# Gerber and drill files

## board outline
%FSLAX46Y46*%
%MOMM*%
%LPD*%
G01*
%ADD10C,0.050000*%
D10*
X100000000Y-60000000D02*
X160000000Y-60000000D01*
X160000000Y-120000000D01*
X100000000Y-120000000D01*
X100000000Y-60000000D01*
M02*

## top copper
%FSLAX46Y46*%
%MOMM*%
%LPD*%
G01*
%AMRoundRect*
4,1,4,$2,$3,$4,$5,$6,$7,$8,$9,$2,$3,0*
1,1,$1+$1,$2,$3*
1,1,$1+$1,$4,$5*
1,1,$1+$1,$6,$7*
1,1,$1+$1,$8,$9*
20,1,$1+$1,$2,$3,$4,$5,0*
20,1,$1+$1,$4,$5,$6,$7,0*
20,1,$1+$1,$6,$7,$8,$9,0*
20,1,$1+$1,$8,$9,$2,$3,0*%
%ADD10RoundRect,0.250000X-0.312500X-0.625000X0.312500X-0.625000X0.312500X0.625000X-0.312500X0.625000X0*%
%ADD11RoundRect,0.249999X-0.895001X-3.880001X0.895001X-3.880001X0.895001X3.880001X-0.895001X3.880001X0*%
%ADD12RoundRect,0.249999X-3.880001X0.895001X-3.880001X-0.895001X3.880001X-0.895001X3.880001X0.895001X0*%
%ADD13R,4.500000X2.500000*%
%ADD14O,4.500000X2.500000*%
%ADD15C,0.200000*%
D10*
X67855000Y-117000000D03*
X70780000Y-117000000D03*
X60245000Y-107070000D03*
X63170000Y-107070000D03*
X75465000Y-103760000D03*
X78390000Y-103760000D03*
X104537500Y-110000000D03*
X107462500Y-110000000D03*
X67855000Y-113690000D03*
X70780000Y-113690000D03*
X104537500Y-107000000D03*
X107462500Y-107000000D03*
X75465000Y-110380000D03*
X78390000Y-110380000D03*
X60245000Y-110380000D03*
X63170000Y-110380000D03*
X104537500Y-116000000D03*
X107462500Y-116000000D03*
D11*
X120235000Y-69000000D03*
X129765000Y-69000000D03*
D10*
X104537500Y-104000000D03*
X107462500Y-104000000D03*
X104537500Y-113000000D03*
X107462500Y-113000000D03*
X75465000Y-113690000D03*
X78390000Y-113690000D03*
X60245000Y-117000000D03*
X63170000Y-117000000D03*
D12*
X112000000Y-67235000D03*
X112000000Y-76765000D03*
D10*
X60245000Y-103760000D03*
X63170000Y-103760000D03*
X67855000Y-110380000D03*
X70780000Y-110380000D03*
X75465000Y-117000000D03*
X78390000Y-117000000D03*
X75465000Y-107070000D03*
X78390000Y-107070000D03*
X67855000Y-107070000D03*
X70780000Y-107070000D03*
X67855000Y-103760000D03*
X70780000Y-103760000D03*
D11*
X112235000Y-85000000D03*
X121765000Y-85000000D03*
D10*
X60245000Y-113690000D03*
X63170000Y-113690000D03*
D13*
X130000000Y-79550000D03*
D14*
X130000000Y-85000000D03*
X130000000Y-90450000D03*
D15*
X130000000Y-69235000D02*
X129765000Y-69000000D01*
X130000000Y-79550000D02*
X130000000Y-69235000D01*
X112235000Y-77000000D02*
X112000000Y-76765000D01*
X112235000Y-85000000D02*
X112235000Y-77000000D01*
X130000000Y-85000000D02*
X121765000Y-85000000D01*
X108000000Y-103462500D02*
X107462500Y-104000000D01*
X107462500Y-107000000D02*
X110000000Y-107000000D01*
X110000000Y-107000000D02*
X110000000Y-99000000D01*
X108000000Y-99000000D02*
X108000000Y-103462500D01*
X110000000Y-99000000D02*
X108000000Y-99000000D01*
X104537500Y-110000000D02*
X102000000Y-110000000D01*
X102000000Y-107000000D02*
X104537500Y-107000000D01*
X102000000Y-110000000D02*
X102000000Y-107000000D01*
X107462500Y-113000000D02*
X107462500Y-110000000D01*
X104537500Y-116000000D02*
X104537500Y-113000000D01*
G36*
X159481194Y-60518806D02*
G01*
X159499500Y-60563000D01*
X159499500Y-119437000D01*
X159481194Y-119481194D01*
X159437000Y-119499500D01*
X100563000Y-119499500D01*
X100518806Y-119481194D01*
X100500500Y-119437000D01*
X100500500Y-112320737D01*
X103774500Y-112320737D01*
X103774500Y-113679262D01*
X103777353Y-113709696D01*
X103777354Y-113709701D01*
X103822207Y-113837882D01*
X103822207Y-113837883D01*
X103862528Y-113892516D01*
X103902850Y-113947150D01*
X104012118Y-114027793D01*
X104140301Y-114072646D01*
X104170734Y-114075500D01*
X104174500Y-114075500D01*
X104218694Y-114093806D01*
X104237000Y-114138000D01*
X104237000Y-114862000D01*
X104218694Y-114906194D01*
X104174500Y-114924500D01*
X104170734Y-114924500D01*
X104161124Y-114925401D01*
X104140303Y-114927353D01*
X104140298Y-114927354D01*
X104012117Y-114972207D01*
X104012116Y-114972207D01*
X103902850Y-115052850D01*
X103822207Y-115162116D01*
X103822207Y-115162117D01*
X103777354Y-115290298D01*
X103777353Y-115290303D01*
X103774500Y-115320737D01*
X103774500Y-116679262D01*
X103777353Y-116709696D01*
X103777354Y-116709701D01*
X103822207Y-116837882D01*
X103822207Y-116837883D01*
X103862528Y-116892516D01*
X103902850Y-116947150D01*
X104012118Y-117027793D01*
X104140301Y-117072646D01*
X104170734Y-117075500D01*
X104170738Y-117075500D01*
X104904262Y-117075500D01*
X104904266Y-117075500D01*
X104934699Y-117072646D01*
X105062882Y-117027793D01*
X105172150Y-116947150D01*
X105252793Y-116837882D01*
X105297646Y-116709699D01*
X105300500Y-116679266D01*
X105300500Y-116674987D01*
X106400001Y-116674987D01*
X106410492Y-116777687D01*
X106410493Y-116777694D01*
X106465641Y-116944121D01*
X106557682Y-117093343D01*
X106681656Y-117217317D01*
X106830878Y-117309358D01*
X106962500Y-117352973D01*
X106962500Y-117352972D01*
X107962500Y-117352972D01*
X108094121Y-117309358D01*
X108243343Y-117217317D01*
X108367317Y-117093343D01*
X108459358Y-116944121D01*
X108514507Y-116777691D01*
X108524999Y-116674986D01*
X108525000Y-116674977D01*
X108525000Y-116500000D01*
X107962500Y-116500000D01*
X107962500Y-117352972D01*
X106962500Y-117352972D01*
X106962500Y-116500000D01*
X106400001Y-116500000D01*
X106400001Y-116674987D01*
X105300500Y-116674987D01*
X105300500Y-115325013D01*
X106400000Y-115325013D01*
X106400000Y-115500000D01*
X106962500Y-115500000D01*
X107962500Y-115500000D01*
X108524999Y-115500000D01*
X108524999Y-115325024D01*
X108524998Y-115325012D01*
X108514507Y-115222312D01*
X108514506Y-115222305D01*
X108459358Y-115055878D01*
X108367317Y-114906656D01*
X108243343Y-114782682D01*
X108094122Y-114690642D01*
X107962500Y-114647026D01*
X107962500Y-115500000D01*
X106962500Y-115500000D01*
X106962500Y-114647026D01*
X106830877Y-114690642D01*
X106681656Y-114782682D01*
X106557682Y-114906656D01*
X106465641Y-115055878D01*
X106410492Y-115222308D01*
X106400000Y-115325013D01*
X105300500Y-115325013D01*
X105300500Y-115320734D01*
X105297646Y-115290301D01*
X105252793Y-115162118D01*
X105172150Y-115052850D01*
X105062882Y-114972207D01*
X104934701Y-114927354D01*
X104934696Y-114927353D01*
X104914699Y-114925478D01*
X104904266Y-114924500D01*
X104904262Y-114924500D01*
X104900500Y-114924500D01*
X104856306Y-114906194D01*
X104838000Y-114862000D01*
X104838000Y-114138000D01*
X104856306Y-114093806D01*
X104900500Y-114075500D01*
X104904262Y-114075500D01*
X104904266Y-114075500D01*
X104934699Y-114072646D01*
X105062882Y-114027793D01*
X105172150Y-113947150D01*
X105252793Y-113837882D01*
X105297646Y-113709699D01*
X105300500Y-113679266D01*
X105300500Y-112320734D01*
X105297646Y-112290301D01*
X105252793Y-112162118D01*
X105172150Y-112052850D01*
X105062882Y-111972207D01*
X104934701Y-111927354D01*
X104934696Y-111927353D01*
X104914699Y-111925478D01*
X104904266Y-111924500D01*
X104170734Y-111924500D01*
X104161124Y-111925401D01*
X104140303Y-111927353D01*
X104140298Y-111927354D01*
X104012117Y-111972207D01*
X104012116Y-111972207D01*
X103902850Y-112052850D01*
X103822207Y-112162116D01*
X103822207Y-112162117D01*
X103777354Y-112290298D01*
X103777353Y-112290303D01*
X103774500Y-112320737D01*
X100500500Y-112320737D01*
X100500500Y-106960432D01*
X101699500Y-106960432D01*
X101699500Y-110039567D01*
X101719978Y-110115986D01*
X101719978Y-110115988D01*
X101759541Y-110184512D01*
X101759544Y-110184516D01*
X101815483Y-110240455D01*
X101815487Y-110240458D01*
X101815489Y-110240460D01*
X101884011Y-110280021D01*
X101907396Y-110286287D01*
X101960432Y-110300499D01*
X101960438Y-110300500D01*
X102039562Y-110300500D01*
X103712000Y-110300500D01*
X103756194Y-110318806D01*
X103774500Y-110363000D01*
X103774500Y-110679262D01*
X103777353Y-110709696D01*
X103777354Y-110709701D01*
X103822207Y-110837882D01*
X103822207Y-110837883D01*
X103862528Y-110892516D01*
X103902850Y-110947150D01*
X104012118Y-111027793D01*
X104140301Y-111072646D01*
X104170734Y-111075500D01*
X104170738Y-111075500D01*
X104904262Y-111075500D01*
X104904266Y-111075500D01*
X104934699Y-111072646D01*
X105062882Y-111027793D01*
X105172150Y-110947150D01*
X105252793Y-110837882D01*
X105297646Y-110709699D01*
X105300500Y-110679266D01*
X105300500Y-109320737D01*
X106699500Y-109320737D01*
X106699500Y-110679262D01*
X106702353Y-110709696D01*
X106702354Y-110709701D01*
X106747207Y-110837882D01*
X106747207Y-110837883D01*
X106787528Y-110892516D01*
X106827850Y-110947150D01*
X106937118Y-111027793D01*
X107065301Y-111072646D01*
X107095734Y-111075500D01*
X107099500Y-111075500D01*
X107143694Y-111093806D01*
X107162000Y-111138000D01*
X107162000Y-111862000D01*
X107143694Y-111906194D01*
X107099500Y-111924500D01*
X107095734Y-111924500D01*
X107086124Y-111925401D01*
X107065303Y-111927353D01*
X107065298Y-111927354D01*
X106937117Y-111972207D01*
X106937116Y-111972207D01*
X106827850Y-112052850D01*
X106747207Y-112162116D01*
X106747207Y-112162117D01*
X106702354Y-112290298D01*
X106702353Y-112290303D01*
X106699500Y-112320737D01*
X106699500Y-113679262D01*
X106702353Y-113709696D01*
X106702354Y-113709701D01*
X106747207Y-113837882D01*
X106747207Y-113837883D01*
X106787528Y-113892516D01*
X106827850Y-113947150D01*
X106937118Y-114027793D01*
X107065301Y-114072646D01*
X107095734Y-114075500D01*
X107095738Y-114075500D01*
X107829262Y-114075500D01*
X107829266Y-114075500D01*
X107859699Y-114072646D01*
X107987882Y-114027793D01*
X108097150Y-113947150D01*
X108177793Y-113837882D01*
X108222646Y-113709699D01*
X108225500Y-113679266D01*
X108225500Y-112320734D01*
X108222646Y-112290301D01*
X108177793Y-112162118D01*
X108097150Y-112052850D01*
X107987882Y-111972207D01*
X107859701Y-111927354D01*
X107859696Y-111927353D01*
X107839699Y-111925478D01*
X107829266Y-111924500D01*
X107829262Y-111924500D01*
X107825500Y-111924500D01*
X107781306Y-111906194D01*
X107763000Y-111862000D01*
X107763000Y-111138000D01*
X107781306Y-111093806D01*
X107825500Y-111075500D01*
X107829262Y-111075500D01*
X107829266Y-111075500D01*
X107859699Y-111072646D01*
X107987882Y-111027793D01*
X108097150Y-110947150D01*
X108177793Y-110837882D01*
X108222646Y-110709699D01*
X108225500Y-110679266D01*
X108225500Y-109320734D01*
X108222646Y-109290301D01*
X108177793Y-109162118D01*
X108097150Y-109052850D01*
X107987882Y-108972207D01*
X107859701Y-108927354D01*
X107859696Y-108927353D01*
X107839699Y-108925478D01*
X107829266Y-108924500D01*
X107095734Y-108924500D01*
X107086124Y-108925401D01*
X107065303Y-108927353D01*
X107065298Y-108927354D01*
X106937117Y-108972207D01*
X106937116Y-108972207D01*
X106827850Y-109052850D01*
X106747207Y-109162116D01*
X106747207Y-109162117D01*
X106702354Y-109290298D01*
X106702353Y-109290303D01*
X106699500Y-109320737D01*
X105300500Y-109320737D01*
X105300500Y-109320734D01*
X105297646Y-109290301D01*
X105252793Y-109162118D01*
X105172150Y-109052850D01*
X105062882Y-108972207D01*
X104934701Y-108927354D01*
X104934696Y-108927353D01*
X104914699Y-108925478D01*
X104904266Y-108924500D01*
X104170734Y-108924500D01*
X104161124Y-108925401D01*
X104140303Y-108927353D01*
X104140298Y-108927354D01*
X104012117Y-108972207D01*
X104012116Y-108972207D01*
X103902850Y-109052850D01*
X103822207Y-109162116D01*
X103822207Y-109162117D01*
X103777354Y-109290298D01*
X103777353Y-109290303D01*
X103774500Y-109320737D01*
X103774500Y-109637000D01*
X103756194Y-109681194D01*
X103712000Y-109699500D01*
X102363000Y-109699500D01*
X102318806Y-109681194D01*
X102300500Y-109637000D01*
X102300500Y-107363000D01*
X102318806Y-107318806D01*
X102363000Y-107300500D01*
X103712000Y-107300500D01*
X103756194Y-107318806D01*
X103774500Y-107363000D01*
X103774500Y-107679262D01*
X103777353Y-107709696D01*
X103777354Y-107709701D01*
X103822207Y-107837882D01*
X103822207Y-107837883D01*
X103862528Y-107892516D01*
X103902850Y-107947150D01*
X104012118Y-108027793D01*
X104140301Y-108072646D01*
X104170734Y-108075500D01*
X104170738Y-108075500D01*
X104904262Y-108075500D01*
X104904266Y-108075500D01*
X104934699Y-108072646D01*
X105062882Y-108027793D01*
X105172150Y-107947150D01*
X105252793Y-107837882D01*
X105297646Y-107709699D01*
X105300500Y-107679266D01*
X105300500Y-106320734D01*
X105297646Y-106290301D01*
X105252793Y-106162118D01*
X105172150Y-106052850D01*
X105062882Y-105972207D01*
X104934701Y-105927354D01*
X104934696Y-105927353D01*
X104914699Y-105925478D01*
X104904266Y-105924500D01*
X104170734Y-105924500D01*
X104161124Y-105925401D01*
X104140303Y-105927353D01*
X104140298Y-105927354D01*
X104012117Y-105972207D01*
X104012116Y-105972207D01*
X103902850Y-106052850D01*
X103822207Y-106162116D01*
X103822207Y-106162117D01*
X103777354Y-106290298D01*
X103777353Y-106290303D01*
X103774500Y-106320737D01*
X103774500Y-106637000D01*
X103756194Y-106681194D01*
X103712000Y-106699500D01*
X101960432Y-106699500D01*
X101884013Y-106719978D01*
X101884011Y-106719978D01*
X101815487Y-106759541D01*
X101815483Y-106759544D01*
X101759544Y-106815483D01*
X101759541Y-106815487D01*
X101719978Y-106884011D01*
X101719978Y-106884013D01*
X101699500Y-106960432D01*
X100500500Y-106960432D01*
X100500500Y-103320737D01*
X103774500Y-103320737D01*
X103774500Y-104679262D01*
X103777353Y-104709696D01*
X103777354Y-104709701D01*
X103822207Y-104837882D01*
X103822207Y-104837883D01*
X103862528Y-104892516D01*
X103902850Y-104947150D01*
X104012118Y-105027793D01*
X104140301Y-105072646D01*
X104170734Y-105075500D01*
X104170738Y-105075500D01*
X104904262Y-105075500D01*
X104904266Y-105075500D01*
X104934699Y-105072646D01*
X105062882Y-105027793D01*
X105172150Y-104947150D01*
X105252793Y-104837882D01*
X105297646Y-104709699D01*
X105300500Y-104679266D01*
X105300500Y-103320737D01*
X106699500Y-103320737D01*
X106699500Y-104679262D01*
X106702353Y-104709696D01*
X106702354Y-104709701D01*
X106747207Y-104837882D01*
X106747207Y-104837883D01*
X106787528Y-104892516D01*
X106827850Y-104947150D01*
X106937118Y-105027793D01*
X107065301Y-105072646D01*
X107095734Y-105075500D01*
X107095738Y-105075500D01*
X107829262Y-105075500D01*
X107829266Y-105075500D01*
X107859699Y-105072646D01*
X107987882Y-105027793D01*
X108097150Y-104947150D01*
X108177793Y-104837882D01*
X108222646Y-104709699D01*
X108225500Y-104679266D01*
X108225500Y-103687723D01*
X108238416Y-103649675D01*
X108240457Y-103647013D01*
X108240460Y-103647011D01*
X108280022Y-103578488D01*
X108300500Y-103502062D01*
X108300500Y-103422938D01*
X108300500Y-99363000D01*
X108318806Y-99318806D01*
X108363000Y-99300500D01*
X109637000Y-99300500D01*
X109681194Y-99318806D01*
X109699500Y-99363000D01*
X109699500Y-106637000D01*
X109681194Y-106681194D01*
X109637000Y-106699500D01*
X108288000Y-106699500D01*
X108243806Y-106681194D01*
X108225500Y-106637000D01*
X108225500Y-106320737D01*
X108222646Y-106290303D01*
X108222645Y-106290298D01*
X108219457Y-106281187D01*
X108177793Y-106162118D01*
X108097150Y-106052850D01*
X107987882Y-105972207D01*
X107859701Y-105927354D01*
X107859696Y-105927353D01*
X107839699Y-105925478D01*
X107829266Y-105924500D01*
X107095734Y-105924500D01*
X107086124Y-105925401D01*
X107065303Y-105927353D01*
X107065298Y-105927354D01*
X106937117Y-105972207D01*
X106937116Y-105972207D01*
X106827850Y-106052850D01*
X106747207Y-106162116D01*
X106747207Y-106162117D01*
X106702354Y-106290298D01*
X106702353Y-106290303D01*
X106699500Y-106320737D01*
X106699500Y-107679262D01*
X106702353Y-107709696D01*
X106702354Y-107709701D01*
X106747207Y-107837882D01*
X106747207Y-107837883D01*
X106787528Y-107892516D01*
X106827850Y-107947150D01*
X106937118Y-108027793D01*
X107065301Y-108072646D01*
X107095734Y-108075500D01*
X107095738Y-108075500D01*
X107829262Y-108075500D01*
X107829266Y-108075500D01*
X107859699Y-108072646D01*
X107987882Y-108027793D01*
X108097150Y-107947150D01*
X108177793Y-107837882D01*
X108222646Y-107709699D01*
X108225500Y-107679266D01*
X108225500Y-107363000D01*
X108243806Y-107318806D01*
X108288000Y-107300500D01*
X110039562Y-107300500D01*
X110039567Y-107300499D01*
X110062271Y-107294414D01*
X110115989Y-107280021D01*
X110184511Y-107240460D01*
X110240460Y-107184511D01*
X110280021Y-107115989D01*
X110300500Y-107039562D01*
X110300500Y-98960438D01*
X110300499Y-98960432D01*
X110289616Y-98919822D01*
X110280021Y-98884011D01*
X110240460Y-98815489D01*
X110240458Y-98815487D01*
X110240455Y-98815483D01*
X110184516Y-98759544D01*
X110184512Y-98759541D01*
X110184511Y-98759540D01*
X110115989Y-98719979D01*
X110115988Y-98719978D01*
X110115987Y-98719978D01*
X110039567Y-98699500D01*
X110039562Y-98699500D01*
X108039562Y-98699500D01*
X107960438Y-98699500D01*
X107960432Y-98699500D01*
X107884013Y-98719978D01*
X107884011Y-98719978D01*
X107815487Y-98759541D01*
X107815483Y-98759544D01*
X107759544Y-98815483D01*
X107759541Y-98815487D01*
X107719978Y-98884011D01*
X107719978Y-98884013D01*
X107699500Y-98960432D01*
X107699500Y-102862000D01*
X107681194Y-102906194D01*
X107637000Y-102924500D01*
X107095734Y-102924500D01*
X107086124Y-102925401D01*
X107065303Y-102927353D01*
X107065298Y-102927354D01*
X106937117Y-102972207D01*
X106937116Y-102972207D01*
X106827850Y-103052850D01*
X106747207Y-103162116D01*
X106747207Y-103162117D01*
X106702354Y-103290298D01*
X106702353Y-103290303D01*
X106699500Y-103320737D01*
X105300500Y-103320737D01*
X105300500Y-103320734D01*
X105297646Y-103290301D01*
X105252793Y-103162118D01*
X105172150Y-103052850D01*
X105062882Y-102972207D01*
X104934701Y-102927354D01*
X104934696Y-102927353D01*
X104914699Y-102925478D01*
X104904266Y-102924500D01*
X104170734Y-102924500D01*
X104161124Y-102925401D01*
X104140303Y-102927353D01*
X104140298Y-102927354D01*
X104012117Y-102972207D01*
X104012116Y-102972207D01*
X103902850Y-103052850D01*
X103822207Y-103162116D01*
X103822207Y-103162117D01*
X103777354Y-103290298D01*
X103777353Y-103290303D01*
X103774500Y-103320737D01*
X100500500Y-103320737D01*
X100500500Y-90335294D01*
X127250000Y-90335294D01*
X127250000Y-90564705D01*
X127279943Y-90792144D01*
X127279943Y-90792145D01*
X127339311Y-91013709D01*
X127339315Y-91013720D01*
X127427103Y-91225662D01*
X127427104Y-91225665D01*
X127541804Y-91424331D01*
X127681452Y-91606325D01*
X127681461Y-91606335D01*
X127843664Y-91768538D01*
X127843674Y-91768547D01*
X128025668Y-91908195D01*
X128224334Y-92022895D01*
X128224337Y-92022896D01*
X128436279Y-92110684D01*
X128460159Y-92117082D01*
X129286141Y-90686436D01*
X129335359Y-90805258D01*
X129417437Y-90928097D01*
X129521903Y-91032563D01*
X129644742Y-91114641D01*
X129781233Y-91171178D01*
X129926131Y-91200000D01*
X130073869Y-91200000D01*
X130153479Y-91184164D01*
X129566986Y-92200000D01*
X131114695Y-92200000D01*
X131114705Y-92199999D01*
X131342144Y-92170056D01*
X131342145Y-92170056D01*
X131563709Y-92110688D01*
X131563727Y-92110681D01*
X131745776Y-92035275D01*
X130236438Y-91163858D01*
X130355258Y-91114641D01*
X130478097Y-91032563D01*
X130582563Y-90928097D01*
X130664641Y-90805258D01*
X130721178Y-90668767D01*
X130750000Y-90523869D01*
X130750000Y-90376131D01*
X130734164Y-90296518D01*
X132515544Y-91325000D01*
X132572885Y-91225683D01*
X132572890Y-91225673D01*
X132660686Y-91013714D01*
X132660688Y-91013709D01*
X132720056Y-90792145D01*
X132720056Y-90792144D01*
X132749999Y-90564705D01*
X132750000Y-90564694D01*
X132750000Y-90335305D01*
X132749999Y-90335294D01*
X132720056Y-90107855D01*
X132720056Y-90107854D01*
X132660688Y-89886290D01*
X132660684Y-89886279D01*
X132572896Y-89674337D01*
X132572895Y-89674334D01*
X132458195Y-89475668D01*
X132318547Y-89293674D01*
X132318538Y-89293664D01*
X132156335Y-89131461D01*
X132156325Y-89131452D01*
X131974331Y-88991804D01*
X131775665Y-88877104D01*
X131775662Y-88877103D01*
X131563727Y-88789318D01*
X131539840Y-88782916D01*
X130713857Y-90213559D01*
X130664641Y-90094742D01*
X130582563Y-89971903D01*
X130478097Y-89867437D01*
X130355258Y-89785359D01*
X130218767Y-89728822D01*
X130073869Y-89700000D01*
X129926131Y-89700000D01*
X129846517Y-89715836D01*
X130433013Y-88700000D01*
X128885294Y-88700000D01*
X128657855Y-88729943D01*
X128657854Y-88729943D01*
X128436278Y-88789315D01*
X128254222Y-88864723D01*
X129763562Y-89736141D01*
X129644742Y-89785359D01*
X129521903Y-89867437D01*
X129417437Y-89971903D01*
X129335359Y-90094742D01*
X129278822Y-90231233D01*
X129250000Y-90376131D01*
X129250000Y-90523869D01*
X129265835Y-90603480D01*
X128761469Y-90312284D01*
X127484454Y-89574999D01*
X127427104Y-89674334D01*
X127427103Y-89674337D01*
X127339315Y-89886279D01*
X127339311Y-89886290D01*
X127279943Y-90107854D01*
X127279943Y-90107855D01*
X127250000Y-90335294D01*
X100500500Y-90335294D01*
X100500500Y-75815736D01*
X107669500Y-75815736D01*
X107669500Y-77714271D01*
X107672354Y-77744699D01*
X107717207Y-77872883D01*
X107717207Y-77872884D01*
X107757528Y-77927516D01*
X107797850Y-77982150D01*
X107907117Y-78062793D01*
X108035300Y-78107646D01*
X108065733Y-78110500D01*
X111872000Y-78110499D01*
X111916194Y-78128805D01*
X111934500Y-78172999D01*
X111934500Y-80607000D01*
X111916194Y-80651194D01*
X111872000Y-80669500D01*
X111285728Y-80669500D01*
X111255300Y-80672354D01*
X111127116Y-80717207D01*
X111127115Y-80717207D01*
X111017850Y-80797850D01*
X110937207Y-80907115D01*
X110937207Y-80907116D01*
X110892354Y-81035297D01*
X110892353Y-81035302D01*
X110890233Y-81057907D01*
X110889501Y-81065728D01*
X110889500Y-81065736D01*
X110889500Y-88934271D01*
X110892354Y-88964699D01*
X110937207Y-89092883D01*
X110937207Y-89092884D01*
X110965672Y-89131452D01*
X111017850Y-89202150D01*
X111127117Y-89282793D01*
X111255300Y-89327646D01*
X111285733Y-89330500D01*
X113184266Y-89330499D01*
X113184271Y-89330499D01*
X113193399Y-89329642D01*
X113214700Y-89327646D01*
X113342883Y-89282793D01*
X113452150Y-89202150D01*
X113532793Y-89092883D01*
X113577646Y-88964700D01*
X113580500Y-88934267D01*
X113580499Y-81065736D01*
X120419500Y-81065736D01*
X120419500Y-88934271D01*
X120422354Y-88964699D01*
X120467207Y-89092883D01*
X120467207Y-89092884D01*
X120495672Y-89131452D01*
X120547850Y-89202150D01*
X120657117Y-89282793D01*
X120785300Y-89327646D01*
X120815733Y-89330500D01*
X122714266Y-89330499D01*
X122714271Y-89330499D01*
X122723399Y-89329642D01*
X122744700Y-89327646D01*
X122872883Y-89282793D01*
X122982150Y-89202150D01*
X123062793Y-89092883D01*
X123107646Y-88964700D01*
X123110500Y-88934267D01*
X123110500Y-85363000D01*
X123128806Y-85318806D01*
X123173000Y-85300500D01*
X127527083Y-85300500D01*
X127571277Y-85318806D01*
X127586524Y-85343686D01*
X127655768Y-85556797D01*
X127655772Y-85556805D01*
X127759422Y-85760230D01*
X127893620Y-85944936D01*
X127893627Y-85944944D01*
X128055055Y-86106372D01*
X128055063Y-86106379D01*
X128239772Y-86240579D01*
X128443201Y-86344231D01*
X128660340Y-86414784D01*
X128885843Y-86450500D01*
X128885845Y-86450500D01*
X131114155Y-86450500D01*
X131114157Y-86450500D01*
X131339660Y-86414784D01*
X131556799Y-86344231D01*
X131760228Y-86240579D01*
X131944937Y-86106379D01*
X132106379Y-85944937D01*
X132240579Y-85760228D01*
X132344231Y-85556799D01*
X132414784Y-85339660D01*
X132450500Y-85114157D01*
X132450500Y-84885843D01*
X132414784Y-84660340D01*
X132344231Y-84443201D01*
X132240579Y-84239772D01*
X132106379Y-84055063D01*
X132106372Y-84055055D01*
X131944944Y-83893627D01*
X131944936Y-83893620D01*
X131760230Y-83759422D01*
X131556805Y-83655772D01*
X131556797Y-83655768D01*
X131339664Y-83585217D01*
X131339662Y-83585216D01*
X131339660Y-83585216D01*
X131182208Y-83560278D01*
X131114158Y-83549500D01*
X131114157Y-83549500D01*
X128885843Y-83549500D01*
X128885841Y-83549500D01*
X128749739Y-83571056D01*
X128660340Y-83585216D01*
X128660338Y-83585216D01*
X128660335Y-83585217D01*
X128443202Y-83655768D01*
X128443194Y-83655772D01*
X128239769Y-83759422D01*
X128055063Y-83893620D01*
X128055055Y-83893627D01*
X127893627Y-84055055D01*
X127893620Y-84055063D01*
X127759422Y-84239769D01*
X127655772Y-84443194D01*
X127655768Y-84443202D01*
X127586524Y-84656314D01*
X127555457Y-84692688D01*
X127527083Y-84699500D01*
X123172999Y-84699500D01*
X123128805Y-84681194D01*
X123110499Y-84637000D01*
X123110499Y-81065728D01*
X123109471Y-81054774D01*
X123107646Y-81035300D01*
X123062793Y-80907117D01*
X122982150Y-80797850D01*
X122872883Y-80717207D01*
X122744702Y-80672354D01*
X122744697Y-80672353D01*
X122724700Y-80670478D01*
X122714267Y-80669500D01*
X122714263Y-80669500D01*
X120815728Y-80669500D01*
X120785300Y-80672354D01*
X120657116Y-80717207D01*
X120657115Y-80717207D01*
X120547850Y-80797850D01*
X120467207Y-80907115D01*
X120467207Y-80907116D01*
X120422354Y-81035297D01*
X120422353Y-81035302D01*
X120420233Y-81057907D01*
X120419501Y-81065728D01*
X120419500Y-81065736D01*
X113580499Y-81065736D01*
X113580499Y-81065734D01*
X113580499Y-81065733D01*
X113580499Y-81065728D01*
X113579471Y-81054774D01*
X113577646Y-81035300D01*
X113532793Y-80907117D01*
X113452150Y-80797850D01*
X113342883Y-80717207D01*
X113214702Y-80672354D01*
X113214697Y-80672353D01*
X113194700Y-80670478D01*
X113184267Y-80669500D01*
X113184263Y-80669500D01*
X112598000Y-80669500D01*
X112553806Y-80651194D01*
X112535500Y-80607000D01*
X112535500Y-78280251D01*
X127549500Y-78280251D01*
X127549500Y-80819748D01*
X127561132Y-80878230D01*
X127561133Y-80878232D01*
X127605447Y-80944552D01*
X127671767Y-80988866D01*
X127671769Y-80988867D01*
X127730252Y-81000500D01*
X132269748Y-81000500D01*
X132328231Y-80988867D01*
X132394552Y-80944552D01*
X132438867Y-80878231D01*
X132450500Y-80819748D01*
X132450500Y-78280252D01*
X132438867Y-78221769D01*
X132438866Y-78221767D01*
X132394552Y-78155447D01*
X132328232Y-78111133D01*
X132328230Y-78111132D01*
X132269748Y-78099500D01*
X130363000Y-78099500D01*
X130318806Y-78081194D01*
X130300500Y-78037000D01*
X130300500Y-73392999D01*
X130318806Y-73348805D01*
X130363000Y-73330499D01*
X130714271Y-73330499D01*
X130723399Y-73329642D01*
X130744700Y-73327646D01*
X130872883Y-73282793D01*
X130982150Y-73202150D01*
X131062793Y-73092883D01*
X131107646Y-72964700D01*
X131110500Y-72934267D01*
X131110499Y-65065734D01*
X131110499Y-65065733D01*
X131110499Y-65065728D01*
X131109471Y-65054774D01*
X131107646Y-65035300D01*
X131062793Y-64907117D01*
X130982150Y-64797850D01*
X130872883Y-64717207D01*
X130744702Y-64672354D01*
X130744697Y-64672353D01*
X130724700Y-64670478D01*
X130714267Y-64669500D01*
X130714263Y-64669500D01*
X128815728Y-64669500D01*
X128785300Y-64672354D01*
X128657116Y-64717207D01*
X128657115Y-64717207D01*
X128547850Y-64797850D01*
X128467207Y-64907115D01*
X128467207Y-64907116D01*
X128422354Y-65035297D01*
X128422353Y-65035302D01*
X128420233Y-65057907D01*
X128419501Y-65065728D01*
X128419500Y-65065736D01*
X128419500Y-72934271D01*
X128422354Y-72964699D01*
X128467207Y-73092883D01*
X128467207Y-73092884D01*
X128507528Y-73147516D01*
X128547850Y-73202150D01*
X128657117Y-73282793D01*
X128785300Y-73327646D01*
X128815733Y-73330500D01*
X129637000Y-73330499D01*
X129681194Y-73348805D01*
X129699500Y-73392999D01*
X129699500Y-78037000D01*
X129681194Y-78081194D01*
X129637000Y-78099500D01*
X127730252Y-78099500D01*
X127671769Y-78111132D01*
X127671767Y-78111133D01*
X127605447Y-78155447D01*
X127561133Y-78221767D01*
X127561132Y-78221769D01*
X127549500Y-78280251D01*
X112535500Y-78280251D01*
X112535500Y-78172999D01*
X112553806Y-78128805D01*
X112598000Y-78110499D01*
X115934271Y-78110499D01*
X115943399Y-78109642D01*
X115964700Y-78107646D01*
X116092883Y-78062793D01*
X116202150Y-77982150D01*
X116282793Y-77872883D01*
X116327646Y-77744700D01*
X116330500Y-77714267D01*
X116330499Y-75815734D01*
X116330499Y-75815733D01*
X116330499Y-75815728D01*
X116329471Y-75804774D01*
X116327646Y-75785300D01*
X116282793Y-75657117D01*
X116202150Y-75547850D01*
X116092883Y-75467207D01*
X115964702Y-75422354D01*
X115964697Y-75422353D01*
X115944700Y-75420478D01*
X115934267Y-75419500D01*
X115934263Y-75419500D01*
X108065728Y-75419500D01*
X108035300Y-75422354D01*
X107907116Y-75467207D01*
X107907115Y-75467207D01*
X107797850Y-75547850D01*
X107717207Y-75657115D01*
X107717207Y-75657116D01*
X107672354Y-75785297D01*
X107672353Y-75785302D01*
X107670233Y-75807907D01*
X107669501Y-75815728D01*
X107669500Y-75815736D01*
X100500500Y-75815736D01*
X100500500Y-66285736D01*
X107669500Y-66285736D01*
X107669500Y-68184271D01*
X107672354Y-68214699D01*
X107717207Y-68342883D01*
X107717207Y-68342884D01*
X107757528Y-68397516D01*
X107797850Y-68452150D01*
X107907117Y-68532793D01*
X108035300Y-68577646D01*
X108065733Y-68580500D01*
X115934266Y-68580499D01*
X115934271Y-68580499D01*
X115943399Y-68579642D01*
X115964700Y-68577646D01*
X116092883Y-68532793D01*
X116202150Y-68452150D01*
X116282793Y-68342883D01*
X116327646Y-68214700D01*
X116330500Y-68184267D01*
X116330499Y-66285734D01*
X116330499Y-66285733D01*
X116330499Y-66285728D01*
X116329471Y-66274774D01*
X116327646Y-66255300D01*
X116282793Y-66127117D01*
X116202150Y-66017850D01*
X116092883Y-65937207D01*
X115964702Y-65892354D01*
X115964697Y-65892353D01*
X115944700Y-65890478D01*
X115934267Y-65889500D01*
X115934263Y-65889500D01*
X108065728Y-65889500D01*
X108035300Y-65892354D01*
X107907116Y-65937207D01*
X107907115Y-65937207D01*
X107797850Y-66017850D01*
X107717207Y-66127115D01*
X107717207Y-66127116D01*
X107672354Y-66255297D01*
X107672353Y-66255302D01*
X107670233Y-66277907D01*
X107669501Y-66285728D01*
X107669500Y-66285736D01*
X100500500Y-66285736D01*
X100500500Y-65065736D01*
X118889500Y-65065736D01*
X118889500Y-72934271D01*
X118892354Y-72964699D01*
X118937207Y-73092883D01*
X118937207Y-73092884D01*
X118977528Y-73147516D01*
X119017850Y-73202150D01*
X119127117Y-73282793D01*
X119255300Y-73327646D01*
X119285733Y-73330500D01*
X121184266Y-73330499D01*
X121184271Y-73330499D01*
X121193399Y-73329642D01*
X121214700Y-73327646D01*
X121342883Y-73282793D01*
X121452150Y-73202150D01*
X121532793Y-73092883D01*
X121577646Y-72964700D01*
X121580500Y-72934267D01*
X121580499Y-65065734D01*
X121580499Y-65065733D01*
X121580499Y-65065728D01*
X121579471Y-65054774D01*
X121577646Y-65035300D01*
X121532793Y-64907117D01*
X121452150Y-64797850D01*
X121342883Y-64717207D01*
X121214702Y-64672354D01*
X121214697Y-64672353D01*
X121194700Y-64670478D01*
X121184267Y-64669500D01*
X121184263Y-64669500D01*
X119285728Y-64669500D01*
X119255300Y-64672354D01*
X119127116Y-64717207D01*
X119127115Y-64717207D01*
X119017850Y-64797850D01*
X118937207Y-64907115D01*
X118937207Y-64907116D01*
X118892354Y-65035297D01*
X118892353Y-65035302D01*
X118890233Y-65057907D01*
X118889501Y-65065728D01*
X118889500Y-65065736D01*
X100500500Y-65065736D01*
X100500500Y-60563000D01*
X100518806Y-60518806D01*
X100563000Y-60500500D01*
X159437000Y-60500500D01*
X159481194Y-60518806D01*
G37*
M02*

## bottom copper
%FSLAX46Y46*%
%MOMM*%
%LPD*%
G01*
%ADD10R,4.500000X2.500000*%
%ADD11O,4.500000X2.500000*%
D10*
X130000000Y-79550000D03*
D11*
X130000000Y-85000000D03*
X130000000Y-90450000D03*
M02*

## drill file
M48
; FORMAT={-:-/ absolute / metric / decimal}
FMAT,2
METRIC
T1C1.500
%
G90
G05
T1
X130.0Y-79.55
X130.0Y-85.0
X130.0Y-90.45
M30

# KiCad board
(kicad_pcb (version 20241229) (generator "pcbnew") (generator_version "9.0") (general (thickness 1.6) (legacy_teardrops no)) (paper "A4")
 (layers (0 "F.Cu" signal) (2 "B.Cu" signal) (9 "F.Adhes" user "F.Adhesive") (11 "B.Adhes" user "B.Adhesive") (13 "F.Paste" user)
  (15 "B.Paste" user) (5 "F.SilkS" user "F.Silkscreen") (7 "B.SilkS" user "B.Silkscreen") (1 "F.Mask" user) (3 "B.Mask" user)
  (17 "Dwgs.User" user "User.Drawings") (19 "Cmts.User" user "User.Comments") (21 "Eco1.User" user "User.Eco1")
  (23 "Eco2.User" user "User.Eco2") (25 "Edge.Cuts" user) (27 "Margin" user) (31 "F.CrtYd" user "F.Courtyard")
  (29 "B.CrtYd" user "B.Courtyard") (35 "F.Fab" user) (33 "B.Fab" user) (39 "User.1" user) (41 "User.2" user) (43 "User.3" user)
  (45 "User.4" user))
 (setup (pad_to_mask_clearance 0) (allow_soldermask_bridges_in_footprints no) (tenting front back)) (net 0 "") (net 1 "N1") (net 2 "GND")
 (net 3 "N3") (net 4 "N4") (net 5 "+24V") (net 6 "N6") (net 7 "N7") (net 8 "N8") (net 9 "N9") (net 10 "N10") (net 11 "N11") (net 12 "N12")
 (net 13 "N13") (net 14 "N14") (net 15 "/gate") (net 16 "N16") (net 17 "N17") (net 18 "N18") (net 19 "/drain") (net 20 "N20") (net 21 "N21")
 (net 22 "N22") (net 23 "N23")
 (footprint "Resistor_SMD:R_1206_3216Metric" (layer "F.Cu") (at 69.3175 117)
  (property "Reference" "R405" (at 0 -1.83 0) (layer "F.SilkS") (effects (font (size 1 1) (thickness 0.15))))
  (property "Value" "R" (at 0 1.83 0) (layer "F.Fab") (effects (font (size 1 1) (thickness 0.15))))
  (pad "1" smd roundrect (at -1.4625 0) (size 1.125 1.75) (layers "F.Cu" "F.Mask" "F.Paste") (roundrect_rratio 0.222222) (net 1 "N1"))
  (pad "2" smd roundrect (at 1.4625 0) (size 1.125 1.75) (layers "F.Cu" "F.Mask" "F.Paste") (roundrect_rratio 0.222222) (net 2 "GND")))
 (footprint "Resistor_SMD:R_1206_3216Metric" (layer "F.Cu") (at 61.7075 107.07)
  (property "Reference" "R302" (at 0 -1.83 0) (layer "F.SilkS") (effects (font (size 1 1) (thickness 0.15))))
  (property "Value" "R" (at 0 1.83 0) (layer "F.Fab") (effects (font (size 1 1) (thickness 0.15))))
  (pad "1" smd roundrect (at -1.4625 0) (size 1.125 1.75) (layers "F.Cu" "F.Mask" "F.Paste") (roundrect_rratio 0.222222) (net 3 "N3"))
  (pad "2" smd roundrect (at 1.4625 0) (size 1.125 1.75) (layers "F.Cu" "F.Mask" "F.Paste") (roundrect_rratio 0.222222) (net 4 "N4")))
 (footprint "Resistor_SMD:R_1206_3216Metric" (layer "F.Cu") (at 76.9275 103.76)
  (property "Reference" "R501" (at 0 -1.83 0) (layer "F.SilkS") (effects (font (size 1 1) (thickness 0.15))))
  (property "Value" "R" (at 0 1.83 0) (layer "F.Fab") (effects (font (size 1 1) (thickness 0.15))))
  (pad "1" smd roundrect (at -1.4625 0) (size 1.125 1.75) (layers "F.Cu" "F.Mask" "F.Paste") (roundrect_rratio 0.222222) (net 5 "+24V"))
  (pad "2" smd roundrect (at 1.4625 0) (size 1.125 1.75) (layers "F.Cu" "F.Mask" "F.Paste") (roundrect_rratio 0.222222) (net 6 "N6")))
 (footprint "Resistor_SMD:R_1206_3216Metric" (layer "F.Cu") (at 106 110)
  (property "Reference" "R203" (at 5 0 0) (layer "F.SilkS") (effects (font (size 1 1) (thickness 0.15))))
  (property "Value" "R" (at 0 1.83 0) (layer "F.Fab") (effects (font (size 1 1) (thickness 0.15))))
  (pad "1" smd roundrect (at -1.4625 0) (size 1.125 1.75) (layers "F.Cu" "F.Mask" "F.Paste") (roundrect_rratio 0.222222) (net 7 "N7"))
  (pad "2" smd roundrect (at 1.4625 0) (size 1.125 1.75) (layers "F.Cu" "F.Mask" "F.Paste") (roundrect_rratio 0.222222) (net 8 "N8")))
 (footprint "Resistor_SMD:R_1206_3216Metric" (layer "F.Cu") (at 69.3175 113.69)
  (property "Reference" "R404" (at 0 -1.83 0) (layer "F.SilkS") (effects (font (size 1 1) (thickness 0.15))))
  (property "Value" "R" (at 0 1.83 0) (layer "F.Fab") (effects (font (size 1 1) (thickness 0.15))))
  (pad "1" smd roundrect (at -1.4625 0) (size 1.125 1.75) (layers "F.Cu" "F.Mask" "F.Paste") (roundrect_rratio 0.222222) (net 1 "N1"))
  (pad "2" smd roundrect (at 1.4625 0) (size 1.125 1.75) (layers "F.Cu" "F.Mask" "F.Paste") (roundrect_rratio 0.222222) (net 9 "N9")))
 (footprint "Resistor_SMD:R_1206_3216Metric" (layer "F.Cu") (at 106 107)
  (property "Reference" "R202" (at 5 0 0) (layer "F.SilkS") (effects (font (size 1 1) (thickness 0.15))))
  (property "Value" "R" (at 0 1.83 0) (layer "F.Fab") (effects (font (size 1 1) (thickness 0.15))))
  (pad "1" smd roundrect (at -1.4625 0) (size 1.125 1.75) (layers "F.Cu" "F.Mask" "F.Paste") (roundrect_rratio 0.222222) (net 7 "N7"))
  (pad "2" smd roundrect (at 1.4625 0) (size 1.125 1.75) (layers "F.Cu" "F.Mask" "F.Paste") (roundrect_rratio 0.222222) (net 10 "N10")))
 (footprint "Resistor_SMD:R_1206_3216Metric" (layer "F.Cu") (at 76.9275 110.38)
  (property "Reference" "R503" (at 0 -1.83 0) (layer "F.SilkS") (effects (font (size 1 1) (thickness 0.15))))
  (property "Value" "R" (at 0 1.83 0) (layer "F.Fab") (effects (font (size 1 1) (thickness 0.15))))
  (pad "1" smd roundrect (at -1.4625 0) (size 1.125 1.75) (layers "F.Cu" "F.Mask" "F.Paste") (roundrect_rratio 0.222222) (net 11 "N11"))
  (pad "2" smd roundrect (at 1.4625 0) (size 1.125 1.75) (layers "F.Cu" "F.Mask" "F.Paste") (roundrect_rratio 0.222222) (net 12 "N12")))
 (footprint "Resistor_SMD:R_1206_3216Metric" (layer "F.Cu") (at 61.7075 110.38)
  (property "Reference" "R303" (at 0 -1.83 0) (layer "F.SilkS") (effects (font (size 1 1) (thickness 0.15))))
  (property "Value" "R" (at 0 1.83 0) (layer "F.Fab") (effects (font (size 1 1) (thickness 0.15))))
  (pad "1" smd roundrect (at -1.4625 0) (size 1.125 1.75) (layers "F.Cu" "F.Mask" "F.Paste") (roundrect_rratio 0.222222) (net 3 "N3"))
  (pad "2" smd roundrect (at 1.4625 0) (size 1.125 1.75) (layers "F.Cu" "F.Mask" "F.Paste") (roundrect_rratio 0.222222) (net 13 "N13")))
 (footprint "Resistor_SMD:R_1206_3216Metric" (layer "F.Cu") (at 106 116)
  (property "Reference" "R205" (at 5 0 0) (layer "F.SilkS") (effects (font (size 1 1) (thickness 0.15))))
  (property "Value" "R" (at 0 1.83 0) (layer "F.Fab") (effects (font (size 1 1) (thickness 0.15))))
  (pad "1" smd roundrect (at -1.4625 0) (size 1.125 1.75) (layers "F.Cu" "F.Mask" "F.Paste") (roundrect_rratio 0.222222) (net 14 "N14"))
  (pad "2" smd roundrect (at 1.4625 0) (size 1.125 1.75) (layers "F.Cu" "F.Mask" "F.Paste") (roundrect_rratio 0.222222) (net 2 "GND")))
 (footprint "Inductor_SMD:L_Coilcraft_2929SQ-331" (layer "F.Cu") (at 125 69)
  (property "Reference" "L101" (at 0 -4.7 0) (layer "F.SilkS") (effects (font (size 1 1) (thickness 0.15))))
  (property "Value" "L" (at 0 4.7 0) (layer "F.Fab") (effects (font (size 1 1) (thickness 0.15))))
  (pad "1" smd roundrect (at -4.765 0) (size 2.29 8.26) (layers "F.Cu" "F.Mask" "F.Paste") (roundrect_rratio 0.10917) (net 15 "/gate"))
  (pad "2" smd roundrect (at 4.765 0) (size 2.29 8.26) (layers "F.Cu" "F.Mask" "F.Paste") (roundrect_rratio 0.10917) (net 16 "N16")))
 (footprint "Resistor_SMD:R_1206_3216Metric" (layer "F.Cu") (at 106 104)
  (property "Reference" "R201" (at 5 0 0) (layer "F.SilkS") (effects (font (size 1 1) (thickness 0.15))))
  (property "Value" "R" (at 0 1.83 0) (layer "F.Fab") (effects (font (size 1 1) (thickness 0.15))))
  (pad "1" smd roundrect (at -1.4625 0) (size 1.125 1.75) (layers "F.Cu" "F.Mask" "F.Paste") (roundrect_rratio 0.222222) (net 5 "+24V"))
  (pad "2" smd roundrect (at 1.4625 0) (size 1.125 1.75) (layers "F.Cu" "F.Mask" "F.Paste") (roundrect_rratio 0.222222) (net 10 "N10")))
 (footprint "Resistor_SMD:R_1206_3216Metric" (layer "F.Cu") (at 106 113)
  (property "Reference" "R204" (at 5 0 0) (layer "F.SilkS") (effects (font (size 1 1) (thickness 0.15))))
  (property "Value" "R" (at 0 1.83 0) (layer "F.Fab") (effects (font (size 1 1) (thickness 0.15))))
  (pad "1" smd roundrect (at -1.4625 0) (size 1.125 1.75) (layers "F.Cu" "F.Mask" "F.Paste") (roundrect_rratio 0.222222) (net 14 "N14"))
  (pad "2" smd roundrect (at 1.4625 0) (size 1.125 1.75) (layers "F.Cu" "F.Mask" "F.Paste") (roundrect_rratio 0.222222) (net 8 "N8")))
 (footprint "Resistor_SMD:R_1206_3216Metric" (layer "F.Cu") (at 76.9275 113.69)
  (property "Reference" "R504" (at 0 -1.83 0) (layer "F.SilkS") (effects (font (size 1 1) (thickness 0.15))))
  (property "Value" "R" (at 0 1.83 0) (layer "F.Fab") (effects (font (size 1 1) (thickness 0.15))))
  (pad "1" smd roundrect (at -1.4625 0) (size 1.125 1.75) (layers "F.Cu" "F.Mask" "F.Paste") (roundrect_rratio 0.222222) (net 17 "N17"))
  (pad "2" smd roundrect (at 1.4625 0) (size 1.125 1.75) (layers "F.Cu" "F.Mask" "F.Paste") (roundrect_rratio 0.222222) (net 12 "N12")))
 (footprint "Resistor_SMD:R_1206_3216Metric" (layer "F.Cu") (at 61.7075 117)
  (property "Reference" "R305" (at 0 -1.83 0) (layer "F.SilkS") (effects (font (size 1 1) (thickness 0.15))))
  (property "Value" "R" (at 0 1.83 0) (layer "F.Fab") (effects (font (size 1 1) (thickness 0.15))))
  (pad "1" smd roundrect (at -1.4625 0) (size 1.125 1.75) (layers "F.Cu" "F.Mask" "F.Paste") (roundrect_rratio 0.222222) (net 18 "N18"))
  (pad "2" smd roundrect (at 1.4625 0) (size 1.125 1.75) (layers "F.Cu" "F.Mask" "F.Paste") (roundrect_rratio 0.222222) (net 2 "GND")))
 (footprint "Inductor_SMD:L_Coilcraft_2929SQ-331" (layer "F.Cu") (at 112 72 -90)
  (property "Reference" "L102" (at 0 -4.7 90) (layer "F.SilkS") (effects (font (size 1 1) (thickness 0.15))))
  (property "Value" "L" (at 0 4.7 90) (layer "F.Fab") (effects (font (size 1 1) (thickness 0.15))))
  (pad "1" smd roundrect (at -4.765 0 270) (size 2.29 8.26) (layers "F.Cu" "F.Mask" "F.Paste") (roundrect_rratio 0.10917) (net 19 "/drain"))
  (pad "2" smd roundrect (at 4.765 0 270) (size 2.29 8.26) (layers "F.Cu" "F.Mask" "F.Paste") (roundrect_rratio 0.10917) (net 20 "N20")))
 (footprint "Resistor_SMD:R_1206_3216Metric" (layer "F.Cu") (at 61.7075 103.76)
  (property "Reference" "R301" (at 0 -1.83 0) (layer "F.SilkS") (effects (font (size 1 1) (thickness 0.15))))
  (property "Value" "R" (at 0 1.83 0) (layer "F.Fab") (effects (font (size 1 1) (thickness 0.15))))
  (pad "1" smd roundrect (at -1.4625 0) (size 1.125 1.75) (layers "F.Cu" "F.Mask" "F.Paste") (roundrect_rratio 0.222222) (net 5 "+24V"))
  (pad "2" smd roundrect (at 1.4625 0) (size 1.125 1.75) (layers "F.Cu" "F.Mask" "F.Paste") (roundrect_rratio 0.222222) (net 4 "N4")))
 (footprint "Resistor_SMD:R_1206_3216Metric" (layer "F.Cu") (at 69.3175 110.38)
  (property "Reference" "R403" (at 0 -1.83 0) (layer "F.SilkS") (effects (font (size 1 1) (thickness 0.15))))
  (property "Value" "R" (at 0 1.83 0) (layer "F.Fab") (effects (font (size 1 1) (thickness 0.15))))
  (pad "1" smd roundrect (at -1.4625 0) (size 1.125 1.75) (layers "F.Cu" "F.Mask" "F.Paste") (roundrect_rratio 0.222222) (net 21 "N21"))
  (pad "2" smd roundrect (at 1.4625 0) (size 1.125 1.75) (layers "F.Cu" "F.Mask" "F.Paste") (roundrect_rratio 0.222222) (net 9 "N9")))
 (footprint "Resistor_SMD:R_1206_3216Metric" (layer "F.Cu") (at 76.9275 117)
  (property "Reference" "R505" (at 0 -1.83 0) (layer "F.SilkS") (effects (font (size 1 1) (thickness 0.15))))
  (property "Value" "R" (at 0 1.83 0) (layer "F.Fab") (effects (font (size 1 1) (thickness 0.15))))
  (pad "1" smd roundrect (at -1.4625 0) (size 1.125 1.75) (layers "F.Cu" "F.Mask" "F.Paste") (roundrect_rratio 0.222222) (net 17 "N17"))
  (pad "2" smd roundrect (at 1.4625 0) (size 1.125 1.75) (layers "F.Cu" "F.Mask" "F.Paste") (roundrect_rratio 0.222222) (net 2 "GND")))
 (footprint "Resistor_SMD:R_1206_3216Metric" (layer "F.Cu") (at 76.9275 107.07)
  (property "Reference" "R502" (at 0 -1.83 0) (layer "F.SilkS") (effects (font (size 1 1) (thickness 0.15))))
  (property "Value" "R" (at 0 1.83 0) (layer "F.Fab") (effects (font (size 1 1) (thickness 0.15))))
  (pad "1" smd roundrect (at -1.4625 0) (size 1.125 1.75) (layers "F.Cu" "F.Mask" "F.Paste") (roundrect_rratio 0.222222) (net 11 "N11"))
  (pad "2" smd roundrect (at 1.4625 0) (size 1.125 1.75) (layers "F.Cu" "F.Mask" "F.Paste") (roundrect_rratio 0.222222) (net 6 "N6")))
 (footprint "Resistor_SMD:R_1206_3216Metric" (layer "F.Cu") (at 69.3175 107.07)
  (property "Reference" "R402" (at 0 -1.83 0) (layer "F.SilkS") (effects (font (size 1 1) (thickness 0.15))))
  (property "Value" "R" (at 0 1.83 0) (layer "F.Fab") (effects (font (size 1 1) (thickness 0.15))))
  (pad "1" smd roundrect (at -1.4625 0) (size 1.125 1.75) (layers "F.Cu" "F.Mask" "F.Paste") (roundrect_rratio 0.222222) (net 21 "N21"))
  (pad "2" smd roundrect (at 1.4625 0) (size 1.125 1.75) (layers "F.Cu" "F.Mask" "F.Paste") (roundrect_rratio 0.222222) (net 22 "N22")))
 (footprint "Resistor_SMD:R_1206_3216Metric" (layer "F.Cu") (at 69.3175 103.76)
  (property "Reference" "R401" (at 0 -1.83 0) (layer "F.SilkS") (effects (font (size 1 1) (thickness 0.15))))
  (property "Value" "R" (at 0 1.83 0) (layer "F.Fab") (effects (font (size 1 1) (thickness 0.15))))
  (pad "1" smd roundrect (at -1.4625 0) (size 1.125 1.75) (layers "F.Cu" "F.Mask" "F.Paste") (roundrect_rratio 0.222222) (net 5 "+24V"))
  (pad "2" smd roundrect (at 1.4625 0) (size 1.125 1.75) (layers "F.Cu" "F.Mask" "F.Paste") (roundrect_rratio 0.222222) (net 22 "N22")))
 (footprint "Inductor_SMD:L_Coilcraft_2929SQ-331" (layer "F.Cu") (at 117 85)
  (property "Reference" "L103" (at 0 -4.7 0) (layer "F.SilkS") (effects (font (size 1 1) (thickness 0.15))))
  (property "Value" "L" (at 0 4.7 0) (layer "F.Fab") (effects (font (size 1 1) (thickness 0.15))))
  (pad "1" smd roundrect (at -4.765 0) (size 2.29 8.26) (layers "F.Cu" "F.Mask" "F.Paste") (roundrect_rratio 0.10917) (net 20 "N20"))
  (pad "2" smd roundrect (at 4.765 0) (size 2.29 8.26) (layers "F.Cu" "F.Mask" "F.Paste") (roundrect_rratio 0.10917) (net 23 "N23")))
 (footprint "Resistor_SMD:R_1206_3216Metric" (layer "F.Cu") (at 61.7075 113.69)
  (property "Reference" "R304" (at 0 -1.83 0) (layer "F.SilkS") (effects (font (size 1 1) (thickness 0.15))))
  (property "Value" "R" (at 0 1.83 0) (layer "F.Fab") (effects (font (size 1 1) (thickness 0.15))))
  (pad "1" smd roundrect (at -1.4625 0) (size 1.125 1.75) (layers "F.Cu" "F.Mask" "F.Paste") (roundrect_rratio 0.222222) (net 18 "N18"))
  (pad "2" smd roundrect (at 1.4625 0) (size 1.125 1.75) (layers "F.Cu" "F.Mask" "F.Paste") (roundrect_rratio 0.222222) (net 13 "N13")))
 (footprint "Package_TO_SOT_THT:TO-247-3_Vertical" (layer "F.Cu") (at 130 79.55 -90)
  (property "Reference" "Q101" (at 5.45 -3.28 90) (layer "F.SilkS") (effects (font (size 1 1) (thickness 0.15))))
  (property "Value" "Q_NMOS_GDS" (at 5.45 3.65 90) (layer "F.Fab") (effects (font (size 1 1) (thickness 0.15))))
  (pad "1" thru_hole rect (at 0 0 270) (size 2.5 4.5) (drill 1.5) (layers "*.Cu" "*.Mask") (remove_unused_layers no) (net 16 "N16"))
  (pad "2" thru_hole oval (at 5.45 0 270) (size 2.5 4.5) (drill 1.5) (layers "*.Cu" "*.Mask") (remove_unused_layers no) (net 23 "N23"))
  (pad "3" thru_hole oval (at 10.9 0 270) (size 2.5 4.5) (drill 1.5) (layers "*.Cu" "*.Mask") (remove_unused_layers no) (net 2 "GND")
   (thermal_bridge_angle 30)))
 (gr_rect (start 100 60) (end 160 120) (stroke (width 0.05) (type default)) (fill no) (layer "Edge.Cuts"))
 (segment (start 130 69.235) (end 129.765 69) (width 0.2) (layer "F.Cu") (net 16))
 (segment (start 130 79.55) (end 130 69.235) (width 0.2) (layer "F.Cu") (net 16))
 (segment (start 112.235 77) (end 112 76.765) (width 0.2) (layer "F.Cu") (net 20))
 (segment (start 112.235 85) (end 112.235 77) (width 0.2) (layer "F.Cu") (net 20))
 (segment (start 130 85) (end 121.765 85) (width 0.2) (layer "F.Cu") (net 23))
 (segment (start 108 103.4625) (end 107.4625 104) (width 0.2) (layer "F.Cu") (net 10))
 (segment (start 107.4625 107) (end 110 107) (width 0.2) (layer "F.Cu") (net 10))
 (segment (start 110 107) (end 110 99) (width 0.2) (layer "F.Cu") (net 10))
 (segment (start 108 99) (end 108 103.4625) (width 0.2) (layer "F.Cu") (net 10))
 (segment (start 110 99) (end 108 99) (width 0.2) (layer "F.Cu") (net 10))
 (segment (start 104.5375 110) (end 102 110) (width 0.2) (layer "F.Cu") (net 7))
 (segment (start 102 107) (end 104.5375 107) (width 0.2) (layer "F.Cu") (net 7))
 (segment (start 102 110) (end 102 107) (width 0.2) (layer "F.Cu") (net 7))
 (segment (start 107.4625 113) (end 107.4625 110) (width 0.2) (layer "F.Cu") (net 8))
 (segment (start 104.5375 116) (end 104.5375 113) (width 0.2) (layer "F.Cu") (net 14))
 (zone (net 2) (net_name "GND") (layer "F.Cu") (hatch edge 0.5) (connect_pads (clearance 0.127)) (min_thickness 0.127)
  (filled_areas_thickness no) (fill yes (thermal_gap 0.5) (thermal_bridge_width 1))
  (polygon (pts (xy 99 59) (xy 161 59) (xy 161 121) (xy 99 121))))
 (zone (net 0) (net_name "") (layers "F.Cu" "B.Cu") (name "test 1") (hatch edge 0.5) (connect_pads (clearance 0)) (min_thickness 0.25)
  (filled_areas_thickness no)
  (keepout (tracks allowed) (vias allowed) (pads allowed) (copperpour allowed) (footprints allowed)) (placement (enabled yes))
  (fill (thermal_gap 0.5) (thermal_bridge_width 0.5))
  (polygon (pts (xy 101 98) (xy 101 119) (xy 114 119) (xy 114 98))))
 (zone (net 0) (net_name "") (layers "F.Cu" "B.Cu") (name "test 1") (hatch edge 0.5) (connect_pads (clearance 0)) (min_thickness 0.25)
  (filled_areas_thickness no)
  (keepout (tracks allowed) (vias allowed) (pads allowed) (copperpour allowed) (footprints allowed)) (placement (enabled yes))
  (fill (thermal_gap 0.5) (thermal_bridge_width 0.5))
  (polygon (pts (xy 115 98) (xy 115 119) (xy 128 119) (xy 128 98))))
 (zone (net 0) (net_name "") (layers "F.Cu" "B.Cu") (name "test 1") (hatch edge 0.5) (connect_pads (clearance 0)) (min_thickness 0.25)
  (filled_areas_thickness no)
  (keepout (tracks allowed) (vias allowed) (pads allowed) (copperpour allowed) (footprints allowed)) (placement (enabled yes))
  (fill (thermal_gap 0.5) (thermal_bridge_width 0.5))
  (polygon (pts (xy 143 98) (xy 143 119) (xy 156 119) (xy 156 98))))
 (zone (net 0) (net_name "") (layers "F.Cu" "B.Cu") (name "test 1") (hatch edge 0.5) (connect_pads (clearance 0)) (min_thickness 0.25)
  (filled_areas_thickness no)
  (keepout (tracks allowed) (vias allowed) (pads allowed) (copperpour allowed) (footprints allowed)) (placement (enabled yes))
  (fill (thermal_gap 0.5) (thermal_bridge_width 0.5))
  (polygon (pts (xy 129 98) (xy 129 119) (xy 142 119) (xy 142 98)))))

